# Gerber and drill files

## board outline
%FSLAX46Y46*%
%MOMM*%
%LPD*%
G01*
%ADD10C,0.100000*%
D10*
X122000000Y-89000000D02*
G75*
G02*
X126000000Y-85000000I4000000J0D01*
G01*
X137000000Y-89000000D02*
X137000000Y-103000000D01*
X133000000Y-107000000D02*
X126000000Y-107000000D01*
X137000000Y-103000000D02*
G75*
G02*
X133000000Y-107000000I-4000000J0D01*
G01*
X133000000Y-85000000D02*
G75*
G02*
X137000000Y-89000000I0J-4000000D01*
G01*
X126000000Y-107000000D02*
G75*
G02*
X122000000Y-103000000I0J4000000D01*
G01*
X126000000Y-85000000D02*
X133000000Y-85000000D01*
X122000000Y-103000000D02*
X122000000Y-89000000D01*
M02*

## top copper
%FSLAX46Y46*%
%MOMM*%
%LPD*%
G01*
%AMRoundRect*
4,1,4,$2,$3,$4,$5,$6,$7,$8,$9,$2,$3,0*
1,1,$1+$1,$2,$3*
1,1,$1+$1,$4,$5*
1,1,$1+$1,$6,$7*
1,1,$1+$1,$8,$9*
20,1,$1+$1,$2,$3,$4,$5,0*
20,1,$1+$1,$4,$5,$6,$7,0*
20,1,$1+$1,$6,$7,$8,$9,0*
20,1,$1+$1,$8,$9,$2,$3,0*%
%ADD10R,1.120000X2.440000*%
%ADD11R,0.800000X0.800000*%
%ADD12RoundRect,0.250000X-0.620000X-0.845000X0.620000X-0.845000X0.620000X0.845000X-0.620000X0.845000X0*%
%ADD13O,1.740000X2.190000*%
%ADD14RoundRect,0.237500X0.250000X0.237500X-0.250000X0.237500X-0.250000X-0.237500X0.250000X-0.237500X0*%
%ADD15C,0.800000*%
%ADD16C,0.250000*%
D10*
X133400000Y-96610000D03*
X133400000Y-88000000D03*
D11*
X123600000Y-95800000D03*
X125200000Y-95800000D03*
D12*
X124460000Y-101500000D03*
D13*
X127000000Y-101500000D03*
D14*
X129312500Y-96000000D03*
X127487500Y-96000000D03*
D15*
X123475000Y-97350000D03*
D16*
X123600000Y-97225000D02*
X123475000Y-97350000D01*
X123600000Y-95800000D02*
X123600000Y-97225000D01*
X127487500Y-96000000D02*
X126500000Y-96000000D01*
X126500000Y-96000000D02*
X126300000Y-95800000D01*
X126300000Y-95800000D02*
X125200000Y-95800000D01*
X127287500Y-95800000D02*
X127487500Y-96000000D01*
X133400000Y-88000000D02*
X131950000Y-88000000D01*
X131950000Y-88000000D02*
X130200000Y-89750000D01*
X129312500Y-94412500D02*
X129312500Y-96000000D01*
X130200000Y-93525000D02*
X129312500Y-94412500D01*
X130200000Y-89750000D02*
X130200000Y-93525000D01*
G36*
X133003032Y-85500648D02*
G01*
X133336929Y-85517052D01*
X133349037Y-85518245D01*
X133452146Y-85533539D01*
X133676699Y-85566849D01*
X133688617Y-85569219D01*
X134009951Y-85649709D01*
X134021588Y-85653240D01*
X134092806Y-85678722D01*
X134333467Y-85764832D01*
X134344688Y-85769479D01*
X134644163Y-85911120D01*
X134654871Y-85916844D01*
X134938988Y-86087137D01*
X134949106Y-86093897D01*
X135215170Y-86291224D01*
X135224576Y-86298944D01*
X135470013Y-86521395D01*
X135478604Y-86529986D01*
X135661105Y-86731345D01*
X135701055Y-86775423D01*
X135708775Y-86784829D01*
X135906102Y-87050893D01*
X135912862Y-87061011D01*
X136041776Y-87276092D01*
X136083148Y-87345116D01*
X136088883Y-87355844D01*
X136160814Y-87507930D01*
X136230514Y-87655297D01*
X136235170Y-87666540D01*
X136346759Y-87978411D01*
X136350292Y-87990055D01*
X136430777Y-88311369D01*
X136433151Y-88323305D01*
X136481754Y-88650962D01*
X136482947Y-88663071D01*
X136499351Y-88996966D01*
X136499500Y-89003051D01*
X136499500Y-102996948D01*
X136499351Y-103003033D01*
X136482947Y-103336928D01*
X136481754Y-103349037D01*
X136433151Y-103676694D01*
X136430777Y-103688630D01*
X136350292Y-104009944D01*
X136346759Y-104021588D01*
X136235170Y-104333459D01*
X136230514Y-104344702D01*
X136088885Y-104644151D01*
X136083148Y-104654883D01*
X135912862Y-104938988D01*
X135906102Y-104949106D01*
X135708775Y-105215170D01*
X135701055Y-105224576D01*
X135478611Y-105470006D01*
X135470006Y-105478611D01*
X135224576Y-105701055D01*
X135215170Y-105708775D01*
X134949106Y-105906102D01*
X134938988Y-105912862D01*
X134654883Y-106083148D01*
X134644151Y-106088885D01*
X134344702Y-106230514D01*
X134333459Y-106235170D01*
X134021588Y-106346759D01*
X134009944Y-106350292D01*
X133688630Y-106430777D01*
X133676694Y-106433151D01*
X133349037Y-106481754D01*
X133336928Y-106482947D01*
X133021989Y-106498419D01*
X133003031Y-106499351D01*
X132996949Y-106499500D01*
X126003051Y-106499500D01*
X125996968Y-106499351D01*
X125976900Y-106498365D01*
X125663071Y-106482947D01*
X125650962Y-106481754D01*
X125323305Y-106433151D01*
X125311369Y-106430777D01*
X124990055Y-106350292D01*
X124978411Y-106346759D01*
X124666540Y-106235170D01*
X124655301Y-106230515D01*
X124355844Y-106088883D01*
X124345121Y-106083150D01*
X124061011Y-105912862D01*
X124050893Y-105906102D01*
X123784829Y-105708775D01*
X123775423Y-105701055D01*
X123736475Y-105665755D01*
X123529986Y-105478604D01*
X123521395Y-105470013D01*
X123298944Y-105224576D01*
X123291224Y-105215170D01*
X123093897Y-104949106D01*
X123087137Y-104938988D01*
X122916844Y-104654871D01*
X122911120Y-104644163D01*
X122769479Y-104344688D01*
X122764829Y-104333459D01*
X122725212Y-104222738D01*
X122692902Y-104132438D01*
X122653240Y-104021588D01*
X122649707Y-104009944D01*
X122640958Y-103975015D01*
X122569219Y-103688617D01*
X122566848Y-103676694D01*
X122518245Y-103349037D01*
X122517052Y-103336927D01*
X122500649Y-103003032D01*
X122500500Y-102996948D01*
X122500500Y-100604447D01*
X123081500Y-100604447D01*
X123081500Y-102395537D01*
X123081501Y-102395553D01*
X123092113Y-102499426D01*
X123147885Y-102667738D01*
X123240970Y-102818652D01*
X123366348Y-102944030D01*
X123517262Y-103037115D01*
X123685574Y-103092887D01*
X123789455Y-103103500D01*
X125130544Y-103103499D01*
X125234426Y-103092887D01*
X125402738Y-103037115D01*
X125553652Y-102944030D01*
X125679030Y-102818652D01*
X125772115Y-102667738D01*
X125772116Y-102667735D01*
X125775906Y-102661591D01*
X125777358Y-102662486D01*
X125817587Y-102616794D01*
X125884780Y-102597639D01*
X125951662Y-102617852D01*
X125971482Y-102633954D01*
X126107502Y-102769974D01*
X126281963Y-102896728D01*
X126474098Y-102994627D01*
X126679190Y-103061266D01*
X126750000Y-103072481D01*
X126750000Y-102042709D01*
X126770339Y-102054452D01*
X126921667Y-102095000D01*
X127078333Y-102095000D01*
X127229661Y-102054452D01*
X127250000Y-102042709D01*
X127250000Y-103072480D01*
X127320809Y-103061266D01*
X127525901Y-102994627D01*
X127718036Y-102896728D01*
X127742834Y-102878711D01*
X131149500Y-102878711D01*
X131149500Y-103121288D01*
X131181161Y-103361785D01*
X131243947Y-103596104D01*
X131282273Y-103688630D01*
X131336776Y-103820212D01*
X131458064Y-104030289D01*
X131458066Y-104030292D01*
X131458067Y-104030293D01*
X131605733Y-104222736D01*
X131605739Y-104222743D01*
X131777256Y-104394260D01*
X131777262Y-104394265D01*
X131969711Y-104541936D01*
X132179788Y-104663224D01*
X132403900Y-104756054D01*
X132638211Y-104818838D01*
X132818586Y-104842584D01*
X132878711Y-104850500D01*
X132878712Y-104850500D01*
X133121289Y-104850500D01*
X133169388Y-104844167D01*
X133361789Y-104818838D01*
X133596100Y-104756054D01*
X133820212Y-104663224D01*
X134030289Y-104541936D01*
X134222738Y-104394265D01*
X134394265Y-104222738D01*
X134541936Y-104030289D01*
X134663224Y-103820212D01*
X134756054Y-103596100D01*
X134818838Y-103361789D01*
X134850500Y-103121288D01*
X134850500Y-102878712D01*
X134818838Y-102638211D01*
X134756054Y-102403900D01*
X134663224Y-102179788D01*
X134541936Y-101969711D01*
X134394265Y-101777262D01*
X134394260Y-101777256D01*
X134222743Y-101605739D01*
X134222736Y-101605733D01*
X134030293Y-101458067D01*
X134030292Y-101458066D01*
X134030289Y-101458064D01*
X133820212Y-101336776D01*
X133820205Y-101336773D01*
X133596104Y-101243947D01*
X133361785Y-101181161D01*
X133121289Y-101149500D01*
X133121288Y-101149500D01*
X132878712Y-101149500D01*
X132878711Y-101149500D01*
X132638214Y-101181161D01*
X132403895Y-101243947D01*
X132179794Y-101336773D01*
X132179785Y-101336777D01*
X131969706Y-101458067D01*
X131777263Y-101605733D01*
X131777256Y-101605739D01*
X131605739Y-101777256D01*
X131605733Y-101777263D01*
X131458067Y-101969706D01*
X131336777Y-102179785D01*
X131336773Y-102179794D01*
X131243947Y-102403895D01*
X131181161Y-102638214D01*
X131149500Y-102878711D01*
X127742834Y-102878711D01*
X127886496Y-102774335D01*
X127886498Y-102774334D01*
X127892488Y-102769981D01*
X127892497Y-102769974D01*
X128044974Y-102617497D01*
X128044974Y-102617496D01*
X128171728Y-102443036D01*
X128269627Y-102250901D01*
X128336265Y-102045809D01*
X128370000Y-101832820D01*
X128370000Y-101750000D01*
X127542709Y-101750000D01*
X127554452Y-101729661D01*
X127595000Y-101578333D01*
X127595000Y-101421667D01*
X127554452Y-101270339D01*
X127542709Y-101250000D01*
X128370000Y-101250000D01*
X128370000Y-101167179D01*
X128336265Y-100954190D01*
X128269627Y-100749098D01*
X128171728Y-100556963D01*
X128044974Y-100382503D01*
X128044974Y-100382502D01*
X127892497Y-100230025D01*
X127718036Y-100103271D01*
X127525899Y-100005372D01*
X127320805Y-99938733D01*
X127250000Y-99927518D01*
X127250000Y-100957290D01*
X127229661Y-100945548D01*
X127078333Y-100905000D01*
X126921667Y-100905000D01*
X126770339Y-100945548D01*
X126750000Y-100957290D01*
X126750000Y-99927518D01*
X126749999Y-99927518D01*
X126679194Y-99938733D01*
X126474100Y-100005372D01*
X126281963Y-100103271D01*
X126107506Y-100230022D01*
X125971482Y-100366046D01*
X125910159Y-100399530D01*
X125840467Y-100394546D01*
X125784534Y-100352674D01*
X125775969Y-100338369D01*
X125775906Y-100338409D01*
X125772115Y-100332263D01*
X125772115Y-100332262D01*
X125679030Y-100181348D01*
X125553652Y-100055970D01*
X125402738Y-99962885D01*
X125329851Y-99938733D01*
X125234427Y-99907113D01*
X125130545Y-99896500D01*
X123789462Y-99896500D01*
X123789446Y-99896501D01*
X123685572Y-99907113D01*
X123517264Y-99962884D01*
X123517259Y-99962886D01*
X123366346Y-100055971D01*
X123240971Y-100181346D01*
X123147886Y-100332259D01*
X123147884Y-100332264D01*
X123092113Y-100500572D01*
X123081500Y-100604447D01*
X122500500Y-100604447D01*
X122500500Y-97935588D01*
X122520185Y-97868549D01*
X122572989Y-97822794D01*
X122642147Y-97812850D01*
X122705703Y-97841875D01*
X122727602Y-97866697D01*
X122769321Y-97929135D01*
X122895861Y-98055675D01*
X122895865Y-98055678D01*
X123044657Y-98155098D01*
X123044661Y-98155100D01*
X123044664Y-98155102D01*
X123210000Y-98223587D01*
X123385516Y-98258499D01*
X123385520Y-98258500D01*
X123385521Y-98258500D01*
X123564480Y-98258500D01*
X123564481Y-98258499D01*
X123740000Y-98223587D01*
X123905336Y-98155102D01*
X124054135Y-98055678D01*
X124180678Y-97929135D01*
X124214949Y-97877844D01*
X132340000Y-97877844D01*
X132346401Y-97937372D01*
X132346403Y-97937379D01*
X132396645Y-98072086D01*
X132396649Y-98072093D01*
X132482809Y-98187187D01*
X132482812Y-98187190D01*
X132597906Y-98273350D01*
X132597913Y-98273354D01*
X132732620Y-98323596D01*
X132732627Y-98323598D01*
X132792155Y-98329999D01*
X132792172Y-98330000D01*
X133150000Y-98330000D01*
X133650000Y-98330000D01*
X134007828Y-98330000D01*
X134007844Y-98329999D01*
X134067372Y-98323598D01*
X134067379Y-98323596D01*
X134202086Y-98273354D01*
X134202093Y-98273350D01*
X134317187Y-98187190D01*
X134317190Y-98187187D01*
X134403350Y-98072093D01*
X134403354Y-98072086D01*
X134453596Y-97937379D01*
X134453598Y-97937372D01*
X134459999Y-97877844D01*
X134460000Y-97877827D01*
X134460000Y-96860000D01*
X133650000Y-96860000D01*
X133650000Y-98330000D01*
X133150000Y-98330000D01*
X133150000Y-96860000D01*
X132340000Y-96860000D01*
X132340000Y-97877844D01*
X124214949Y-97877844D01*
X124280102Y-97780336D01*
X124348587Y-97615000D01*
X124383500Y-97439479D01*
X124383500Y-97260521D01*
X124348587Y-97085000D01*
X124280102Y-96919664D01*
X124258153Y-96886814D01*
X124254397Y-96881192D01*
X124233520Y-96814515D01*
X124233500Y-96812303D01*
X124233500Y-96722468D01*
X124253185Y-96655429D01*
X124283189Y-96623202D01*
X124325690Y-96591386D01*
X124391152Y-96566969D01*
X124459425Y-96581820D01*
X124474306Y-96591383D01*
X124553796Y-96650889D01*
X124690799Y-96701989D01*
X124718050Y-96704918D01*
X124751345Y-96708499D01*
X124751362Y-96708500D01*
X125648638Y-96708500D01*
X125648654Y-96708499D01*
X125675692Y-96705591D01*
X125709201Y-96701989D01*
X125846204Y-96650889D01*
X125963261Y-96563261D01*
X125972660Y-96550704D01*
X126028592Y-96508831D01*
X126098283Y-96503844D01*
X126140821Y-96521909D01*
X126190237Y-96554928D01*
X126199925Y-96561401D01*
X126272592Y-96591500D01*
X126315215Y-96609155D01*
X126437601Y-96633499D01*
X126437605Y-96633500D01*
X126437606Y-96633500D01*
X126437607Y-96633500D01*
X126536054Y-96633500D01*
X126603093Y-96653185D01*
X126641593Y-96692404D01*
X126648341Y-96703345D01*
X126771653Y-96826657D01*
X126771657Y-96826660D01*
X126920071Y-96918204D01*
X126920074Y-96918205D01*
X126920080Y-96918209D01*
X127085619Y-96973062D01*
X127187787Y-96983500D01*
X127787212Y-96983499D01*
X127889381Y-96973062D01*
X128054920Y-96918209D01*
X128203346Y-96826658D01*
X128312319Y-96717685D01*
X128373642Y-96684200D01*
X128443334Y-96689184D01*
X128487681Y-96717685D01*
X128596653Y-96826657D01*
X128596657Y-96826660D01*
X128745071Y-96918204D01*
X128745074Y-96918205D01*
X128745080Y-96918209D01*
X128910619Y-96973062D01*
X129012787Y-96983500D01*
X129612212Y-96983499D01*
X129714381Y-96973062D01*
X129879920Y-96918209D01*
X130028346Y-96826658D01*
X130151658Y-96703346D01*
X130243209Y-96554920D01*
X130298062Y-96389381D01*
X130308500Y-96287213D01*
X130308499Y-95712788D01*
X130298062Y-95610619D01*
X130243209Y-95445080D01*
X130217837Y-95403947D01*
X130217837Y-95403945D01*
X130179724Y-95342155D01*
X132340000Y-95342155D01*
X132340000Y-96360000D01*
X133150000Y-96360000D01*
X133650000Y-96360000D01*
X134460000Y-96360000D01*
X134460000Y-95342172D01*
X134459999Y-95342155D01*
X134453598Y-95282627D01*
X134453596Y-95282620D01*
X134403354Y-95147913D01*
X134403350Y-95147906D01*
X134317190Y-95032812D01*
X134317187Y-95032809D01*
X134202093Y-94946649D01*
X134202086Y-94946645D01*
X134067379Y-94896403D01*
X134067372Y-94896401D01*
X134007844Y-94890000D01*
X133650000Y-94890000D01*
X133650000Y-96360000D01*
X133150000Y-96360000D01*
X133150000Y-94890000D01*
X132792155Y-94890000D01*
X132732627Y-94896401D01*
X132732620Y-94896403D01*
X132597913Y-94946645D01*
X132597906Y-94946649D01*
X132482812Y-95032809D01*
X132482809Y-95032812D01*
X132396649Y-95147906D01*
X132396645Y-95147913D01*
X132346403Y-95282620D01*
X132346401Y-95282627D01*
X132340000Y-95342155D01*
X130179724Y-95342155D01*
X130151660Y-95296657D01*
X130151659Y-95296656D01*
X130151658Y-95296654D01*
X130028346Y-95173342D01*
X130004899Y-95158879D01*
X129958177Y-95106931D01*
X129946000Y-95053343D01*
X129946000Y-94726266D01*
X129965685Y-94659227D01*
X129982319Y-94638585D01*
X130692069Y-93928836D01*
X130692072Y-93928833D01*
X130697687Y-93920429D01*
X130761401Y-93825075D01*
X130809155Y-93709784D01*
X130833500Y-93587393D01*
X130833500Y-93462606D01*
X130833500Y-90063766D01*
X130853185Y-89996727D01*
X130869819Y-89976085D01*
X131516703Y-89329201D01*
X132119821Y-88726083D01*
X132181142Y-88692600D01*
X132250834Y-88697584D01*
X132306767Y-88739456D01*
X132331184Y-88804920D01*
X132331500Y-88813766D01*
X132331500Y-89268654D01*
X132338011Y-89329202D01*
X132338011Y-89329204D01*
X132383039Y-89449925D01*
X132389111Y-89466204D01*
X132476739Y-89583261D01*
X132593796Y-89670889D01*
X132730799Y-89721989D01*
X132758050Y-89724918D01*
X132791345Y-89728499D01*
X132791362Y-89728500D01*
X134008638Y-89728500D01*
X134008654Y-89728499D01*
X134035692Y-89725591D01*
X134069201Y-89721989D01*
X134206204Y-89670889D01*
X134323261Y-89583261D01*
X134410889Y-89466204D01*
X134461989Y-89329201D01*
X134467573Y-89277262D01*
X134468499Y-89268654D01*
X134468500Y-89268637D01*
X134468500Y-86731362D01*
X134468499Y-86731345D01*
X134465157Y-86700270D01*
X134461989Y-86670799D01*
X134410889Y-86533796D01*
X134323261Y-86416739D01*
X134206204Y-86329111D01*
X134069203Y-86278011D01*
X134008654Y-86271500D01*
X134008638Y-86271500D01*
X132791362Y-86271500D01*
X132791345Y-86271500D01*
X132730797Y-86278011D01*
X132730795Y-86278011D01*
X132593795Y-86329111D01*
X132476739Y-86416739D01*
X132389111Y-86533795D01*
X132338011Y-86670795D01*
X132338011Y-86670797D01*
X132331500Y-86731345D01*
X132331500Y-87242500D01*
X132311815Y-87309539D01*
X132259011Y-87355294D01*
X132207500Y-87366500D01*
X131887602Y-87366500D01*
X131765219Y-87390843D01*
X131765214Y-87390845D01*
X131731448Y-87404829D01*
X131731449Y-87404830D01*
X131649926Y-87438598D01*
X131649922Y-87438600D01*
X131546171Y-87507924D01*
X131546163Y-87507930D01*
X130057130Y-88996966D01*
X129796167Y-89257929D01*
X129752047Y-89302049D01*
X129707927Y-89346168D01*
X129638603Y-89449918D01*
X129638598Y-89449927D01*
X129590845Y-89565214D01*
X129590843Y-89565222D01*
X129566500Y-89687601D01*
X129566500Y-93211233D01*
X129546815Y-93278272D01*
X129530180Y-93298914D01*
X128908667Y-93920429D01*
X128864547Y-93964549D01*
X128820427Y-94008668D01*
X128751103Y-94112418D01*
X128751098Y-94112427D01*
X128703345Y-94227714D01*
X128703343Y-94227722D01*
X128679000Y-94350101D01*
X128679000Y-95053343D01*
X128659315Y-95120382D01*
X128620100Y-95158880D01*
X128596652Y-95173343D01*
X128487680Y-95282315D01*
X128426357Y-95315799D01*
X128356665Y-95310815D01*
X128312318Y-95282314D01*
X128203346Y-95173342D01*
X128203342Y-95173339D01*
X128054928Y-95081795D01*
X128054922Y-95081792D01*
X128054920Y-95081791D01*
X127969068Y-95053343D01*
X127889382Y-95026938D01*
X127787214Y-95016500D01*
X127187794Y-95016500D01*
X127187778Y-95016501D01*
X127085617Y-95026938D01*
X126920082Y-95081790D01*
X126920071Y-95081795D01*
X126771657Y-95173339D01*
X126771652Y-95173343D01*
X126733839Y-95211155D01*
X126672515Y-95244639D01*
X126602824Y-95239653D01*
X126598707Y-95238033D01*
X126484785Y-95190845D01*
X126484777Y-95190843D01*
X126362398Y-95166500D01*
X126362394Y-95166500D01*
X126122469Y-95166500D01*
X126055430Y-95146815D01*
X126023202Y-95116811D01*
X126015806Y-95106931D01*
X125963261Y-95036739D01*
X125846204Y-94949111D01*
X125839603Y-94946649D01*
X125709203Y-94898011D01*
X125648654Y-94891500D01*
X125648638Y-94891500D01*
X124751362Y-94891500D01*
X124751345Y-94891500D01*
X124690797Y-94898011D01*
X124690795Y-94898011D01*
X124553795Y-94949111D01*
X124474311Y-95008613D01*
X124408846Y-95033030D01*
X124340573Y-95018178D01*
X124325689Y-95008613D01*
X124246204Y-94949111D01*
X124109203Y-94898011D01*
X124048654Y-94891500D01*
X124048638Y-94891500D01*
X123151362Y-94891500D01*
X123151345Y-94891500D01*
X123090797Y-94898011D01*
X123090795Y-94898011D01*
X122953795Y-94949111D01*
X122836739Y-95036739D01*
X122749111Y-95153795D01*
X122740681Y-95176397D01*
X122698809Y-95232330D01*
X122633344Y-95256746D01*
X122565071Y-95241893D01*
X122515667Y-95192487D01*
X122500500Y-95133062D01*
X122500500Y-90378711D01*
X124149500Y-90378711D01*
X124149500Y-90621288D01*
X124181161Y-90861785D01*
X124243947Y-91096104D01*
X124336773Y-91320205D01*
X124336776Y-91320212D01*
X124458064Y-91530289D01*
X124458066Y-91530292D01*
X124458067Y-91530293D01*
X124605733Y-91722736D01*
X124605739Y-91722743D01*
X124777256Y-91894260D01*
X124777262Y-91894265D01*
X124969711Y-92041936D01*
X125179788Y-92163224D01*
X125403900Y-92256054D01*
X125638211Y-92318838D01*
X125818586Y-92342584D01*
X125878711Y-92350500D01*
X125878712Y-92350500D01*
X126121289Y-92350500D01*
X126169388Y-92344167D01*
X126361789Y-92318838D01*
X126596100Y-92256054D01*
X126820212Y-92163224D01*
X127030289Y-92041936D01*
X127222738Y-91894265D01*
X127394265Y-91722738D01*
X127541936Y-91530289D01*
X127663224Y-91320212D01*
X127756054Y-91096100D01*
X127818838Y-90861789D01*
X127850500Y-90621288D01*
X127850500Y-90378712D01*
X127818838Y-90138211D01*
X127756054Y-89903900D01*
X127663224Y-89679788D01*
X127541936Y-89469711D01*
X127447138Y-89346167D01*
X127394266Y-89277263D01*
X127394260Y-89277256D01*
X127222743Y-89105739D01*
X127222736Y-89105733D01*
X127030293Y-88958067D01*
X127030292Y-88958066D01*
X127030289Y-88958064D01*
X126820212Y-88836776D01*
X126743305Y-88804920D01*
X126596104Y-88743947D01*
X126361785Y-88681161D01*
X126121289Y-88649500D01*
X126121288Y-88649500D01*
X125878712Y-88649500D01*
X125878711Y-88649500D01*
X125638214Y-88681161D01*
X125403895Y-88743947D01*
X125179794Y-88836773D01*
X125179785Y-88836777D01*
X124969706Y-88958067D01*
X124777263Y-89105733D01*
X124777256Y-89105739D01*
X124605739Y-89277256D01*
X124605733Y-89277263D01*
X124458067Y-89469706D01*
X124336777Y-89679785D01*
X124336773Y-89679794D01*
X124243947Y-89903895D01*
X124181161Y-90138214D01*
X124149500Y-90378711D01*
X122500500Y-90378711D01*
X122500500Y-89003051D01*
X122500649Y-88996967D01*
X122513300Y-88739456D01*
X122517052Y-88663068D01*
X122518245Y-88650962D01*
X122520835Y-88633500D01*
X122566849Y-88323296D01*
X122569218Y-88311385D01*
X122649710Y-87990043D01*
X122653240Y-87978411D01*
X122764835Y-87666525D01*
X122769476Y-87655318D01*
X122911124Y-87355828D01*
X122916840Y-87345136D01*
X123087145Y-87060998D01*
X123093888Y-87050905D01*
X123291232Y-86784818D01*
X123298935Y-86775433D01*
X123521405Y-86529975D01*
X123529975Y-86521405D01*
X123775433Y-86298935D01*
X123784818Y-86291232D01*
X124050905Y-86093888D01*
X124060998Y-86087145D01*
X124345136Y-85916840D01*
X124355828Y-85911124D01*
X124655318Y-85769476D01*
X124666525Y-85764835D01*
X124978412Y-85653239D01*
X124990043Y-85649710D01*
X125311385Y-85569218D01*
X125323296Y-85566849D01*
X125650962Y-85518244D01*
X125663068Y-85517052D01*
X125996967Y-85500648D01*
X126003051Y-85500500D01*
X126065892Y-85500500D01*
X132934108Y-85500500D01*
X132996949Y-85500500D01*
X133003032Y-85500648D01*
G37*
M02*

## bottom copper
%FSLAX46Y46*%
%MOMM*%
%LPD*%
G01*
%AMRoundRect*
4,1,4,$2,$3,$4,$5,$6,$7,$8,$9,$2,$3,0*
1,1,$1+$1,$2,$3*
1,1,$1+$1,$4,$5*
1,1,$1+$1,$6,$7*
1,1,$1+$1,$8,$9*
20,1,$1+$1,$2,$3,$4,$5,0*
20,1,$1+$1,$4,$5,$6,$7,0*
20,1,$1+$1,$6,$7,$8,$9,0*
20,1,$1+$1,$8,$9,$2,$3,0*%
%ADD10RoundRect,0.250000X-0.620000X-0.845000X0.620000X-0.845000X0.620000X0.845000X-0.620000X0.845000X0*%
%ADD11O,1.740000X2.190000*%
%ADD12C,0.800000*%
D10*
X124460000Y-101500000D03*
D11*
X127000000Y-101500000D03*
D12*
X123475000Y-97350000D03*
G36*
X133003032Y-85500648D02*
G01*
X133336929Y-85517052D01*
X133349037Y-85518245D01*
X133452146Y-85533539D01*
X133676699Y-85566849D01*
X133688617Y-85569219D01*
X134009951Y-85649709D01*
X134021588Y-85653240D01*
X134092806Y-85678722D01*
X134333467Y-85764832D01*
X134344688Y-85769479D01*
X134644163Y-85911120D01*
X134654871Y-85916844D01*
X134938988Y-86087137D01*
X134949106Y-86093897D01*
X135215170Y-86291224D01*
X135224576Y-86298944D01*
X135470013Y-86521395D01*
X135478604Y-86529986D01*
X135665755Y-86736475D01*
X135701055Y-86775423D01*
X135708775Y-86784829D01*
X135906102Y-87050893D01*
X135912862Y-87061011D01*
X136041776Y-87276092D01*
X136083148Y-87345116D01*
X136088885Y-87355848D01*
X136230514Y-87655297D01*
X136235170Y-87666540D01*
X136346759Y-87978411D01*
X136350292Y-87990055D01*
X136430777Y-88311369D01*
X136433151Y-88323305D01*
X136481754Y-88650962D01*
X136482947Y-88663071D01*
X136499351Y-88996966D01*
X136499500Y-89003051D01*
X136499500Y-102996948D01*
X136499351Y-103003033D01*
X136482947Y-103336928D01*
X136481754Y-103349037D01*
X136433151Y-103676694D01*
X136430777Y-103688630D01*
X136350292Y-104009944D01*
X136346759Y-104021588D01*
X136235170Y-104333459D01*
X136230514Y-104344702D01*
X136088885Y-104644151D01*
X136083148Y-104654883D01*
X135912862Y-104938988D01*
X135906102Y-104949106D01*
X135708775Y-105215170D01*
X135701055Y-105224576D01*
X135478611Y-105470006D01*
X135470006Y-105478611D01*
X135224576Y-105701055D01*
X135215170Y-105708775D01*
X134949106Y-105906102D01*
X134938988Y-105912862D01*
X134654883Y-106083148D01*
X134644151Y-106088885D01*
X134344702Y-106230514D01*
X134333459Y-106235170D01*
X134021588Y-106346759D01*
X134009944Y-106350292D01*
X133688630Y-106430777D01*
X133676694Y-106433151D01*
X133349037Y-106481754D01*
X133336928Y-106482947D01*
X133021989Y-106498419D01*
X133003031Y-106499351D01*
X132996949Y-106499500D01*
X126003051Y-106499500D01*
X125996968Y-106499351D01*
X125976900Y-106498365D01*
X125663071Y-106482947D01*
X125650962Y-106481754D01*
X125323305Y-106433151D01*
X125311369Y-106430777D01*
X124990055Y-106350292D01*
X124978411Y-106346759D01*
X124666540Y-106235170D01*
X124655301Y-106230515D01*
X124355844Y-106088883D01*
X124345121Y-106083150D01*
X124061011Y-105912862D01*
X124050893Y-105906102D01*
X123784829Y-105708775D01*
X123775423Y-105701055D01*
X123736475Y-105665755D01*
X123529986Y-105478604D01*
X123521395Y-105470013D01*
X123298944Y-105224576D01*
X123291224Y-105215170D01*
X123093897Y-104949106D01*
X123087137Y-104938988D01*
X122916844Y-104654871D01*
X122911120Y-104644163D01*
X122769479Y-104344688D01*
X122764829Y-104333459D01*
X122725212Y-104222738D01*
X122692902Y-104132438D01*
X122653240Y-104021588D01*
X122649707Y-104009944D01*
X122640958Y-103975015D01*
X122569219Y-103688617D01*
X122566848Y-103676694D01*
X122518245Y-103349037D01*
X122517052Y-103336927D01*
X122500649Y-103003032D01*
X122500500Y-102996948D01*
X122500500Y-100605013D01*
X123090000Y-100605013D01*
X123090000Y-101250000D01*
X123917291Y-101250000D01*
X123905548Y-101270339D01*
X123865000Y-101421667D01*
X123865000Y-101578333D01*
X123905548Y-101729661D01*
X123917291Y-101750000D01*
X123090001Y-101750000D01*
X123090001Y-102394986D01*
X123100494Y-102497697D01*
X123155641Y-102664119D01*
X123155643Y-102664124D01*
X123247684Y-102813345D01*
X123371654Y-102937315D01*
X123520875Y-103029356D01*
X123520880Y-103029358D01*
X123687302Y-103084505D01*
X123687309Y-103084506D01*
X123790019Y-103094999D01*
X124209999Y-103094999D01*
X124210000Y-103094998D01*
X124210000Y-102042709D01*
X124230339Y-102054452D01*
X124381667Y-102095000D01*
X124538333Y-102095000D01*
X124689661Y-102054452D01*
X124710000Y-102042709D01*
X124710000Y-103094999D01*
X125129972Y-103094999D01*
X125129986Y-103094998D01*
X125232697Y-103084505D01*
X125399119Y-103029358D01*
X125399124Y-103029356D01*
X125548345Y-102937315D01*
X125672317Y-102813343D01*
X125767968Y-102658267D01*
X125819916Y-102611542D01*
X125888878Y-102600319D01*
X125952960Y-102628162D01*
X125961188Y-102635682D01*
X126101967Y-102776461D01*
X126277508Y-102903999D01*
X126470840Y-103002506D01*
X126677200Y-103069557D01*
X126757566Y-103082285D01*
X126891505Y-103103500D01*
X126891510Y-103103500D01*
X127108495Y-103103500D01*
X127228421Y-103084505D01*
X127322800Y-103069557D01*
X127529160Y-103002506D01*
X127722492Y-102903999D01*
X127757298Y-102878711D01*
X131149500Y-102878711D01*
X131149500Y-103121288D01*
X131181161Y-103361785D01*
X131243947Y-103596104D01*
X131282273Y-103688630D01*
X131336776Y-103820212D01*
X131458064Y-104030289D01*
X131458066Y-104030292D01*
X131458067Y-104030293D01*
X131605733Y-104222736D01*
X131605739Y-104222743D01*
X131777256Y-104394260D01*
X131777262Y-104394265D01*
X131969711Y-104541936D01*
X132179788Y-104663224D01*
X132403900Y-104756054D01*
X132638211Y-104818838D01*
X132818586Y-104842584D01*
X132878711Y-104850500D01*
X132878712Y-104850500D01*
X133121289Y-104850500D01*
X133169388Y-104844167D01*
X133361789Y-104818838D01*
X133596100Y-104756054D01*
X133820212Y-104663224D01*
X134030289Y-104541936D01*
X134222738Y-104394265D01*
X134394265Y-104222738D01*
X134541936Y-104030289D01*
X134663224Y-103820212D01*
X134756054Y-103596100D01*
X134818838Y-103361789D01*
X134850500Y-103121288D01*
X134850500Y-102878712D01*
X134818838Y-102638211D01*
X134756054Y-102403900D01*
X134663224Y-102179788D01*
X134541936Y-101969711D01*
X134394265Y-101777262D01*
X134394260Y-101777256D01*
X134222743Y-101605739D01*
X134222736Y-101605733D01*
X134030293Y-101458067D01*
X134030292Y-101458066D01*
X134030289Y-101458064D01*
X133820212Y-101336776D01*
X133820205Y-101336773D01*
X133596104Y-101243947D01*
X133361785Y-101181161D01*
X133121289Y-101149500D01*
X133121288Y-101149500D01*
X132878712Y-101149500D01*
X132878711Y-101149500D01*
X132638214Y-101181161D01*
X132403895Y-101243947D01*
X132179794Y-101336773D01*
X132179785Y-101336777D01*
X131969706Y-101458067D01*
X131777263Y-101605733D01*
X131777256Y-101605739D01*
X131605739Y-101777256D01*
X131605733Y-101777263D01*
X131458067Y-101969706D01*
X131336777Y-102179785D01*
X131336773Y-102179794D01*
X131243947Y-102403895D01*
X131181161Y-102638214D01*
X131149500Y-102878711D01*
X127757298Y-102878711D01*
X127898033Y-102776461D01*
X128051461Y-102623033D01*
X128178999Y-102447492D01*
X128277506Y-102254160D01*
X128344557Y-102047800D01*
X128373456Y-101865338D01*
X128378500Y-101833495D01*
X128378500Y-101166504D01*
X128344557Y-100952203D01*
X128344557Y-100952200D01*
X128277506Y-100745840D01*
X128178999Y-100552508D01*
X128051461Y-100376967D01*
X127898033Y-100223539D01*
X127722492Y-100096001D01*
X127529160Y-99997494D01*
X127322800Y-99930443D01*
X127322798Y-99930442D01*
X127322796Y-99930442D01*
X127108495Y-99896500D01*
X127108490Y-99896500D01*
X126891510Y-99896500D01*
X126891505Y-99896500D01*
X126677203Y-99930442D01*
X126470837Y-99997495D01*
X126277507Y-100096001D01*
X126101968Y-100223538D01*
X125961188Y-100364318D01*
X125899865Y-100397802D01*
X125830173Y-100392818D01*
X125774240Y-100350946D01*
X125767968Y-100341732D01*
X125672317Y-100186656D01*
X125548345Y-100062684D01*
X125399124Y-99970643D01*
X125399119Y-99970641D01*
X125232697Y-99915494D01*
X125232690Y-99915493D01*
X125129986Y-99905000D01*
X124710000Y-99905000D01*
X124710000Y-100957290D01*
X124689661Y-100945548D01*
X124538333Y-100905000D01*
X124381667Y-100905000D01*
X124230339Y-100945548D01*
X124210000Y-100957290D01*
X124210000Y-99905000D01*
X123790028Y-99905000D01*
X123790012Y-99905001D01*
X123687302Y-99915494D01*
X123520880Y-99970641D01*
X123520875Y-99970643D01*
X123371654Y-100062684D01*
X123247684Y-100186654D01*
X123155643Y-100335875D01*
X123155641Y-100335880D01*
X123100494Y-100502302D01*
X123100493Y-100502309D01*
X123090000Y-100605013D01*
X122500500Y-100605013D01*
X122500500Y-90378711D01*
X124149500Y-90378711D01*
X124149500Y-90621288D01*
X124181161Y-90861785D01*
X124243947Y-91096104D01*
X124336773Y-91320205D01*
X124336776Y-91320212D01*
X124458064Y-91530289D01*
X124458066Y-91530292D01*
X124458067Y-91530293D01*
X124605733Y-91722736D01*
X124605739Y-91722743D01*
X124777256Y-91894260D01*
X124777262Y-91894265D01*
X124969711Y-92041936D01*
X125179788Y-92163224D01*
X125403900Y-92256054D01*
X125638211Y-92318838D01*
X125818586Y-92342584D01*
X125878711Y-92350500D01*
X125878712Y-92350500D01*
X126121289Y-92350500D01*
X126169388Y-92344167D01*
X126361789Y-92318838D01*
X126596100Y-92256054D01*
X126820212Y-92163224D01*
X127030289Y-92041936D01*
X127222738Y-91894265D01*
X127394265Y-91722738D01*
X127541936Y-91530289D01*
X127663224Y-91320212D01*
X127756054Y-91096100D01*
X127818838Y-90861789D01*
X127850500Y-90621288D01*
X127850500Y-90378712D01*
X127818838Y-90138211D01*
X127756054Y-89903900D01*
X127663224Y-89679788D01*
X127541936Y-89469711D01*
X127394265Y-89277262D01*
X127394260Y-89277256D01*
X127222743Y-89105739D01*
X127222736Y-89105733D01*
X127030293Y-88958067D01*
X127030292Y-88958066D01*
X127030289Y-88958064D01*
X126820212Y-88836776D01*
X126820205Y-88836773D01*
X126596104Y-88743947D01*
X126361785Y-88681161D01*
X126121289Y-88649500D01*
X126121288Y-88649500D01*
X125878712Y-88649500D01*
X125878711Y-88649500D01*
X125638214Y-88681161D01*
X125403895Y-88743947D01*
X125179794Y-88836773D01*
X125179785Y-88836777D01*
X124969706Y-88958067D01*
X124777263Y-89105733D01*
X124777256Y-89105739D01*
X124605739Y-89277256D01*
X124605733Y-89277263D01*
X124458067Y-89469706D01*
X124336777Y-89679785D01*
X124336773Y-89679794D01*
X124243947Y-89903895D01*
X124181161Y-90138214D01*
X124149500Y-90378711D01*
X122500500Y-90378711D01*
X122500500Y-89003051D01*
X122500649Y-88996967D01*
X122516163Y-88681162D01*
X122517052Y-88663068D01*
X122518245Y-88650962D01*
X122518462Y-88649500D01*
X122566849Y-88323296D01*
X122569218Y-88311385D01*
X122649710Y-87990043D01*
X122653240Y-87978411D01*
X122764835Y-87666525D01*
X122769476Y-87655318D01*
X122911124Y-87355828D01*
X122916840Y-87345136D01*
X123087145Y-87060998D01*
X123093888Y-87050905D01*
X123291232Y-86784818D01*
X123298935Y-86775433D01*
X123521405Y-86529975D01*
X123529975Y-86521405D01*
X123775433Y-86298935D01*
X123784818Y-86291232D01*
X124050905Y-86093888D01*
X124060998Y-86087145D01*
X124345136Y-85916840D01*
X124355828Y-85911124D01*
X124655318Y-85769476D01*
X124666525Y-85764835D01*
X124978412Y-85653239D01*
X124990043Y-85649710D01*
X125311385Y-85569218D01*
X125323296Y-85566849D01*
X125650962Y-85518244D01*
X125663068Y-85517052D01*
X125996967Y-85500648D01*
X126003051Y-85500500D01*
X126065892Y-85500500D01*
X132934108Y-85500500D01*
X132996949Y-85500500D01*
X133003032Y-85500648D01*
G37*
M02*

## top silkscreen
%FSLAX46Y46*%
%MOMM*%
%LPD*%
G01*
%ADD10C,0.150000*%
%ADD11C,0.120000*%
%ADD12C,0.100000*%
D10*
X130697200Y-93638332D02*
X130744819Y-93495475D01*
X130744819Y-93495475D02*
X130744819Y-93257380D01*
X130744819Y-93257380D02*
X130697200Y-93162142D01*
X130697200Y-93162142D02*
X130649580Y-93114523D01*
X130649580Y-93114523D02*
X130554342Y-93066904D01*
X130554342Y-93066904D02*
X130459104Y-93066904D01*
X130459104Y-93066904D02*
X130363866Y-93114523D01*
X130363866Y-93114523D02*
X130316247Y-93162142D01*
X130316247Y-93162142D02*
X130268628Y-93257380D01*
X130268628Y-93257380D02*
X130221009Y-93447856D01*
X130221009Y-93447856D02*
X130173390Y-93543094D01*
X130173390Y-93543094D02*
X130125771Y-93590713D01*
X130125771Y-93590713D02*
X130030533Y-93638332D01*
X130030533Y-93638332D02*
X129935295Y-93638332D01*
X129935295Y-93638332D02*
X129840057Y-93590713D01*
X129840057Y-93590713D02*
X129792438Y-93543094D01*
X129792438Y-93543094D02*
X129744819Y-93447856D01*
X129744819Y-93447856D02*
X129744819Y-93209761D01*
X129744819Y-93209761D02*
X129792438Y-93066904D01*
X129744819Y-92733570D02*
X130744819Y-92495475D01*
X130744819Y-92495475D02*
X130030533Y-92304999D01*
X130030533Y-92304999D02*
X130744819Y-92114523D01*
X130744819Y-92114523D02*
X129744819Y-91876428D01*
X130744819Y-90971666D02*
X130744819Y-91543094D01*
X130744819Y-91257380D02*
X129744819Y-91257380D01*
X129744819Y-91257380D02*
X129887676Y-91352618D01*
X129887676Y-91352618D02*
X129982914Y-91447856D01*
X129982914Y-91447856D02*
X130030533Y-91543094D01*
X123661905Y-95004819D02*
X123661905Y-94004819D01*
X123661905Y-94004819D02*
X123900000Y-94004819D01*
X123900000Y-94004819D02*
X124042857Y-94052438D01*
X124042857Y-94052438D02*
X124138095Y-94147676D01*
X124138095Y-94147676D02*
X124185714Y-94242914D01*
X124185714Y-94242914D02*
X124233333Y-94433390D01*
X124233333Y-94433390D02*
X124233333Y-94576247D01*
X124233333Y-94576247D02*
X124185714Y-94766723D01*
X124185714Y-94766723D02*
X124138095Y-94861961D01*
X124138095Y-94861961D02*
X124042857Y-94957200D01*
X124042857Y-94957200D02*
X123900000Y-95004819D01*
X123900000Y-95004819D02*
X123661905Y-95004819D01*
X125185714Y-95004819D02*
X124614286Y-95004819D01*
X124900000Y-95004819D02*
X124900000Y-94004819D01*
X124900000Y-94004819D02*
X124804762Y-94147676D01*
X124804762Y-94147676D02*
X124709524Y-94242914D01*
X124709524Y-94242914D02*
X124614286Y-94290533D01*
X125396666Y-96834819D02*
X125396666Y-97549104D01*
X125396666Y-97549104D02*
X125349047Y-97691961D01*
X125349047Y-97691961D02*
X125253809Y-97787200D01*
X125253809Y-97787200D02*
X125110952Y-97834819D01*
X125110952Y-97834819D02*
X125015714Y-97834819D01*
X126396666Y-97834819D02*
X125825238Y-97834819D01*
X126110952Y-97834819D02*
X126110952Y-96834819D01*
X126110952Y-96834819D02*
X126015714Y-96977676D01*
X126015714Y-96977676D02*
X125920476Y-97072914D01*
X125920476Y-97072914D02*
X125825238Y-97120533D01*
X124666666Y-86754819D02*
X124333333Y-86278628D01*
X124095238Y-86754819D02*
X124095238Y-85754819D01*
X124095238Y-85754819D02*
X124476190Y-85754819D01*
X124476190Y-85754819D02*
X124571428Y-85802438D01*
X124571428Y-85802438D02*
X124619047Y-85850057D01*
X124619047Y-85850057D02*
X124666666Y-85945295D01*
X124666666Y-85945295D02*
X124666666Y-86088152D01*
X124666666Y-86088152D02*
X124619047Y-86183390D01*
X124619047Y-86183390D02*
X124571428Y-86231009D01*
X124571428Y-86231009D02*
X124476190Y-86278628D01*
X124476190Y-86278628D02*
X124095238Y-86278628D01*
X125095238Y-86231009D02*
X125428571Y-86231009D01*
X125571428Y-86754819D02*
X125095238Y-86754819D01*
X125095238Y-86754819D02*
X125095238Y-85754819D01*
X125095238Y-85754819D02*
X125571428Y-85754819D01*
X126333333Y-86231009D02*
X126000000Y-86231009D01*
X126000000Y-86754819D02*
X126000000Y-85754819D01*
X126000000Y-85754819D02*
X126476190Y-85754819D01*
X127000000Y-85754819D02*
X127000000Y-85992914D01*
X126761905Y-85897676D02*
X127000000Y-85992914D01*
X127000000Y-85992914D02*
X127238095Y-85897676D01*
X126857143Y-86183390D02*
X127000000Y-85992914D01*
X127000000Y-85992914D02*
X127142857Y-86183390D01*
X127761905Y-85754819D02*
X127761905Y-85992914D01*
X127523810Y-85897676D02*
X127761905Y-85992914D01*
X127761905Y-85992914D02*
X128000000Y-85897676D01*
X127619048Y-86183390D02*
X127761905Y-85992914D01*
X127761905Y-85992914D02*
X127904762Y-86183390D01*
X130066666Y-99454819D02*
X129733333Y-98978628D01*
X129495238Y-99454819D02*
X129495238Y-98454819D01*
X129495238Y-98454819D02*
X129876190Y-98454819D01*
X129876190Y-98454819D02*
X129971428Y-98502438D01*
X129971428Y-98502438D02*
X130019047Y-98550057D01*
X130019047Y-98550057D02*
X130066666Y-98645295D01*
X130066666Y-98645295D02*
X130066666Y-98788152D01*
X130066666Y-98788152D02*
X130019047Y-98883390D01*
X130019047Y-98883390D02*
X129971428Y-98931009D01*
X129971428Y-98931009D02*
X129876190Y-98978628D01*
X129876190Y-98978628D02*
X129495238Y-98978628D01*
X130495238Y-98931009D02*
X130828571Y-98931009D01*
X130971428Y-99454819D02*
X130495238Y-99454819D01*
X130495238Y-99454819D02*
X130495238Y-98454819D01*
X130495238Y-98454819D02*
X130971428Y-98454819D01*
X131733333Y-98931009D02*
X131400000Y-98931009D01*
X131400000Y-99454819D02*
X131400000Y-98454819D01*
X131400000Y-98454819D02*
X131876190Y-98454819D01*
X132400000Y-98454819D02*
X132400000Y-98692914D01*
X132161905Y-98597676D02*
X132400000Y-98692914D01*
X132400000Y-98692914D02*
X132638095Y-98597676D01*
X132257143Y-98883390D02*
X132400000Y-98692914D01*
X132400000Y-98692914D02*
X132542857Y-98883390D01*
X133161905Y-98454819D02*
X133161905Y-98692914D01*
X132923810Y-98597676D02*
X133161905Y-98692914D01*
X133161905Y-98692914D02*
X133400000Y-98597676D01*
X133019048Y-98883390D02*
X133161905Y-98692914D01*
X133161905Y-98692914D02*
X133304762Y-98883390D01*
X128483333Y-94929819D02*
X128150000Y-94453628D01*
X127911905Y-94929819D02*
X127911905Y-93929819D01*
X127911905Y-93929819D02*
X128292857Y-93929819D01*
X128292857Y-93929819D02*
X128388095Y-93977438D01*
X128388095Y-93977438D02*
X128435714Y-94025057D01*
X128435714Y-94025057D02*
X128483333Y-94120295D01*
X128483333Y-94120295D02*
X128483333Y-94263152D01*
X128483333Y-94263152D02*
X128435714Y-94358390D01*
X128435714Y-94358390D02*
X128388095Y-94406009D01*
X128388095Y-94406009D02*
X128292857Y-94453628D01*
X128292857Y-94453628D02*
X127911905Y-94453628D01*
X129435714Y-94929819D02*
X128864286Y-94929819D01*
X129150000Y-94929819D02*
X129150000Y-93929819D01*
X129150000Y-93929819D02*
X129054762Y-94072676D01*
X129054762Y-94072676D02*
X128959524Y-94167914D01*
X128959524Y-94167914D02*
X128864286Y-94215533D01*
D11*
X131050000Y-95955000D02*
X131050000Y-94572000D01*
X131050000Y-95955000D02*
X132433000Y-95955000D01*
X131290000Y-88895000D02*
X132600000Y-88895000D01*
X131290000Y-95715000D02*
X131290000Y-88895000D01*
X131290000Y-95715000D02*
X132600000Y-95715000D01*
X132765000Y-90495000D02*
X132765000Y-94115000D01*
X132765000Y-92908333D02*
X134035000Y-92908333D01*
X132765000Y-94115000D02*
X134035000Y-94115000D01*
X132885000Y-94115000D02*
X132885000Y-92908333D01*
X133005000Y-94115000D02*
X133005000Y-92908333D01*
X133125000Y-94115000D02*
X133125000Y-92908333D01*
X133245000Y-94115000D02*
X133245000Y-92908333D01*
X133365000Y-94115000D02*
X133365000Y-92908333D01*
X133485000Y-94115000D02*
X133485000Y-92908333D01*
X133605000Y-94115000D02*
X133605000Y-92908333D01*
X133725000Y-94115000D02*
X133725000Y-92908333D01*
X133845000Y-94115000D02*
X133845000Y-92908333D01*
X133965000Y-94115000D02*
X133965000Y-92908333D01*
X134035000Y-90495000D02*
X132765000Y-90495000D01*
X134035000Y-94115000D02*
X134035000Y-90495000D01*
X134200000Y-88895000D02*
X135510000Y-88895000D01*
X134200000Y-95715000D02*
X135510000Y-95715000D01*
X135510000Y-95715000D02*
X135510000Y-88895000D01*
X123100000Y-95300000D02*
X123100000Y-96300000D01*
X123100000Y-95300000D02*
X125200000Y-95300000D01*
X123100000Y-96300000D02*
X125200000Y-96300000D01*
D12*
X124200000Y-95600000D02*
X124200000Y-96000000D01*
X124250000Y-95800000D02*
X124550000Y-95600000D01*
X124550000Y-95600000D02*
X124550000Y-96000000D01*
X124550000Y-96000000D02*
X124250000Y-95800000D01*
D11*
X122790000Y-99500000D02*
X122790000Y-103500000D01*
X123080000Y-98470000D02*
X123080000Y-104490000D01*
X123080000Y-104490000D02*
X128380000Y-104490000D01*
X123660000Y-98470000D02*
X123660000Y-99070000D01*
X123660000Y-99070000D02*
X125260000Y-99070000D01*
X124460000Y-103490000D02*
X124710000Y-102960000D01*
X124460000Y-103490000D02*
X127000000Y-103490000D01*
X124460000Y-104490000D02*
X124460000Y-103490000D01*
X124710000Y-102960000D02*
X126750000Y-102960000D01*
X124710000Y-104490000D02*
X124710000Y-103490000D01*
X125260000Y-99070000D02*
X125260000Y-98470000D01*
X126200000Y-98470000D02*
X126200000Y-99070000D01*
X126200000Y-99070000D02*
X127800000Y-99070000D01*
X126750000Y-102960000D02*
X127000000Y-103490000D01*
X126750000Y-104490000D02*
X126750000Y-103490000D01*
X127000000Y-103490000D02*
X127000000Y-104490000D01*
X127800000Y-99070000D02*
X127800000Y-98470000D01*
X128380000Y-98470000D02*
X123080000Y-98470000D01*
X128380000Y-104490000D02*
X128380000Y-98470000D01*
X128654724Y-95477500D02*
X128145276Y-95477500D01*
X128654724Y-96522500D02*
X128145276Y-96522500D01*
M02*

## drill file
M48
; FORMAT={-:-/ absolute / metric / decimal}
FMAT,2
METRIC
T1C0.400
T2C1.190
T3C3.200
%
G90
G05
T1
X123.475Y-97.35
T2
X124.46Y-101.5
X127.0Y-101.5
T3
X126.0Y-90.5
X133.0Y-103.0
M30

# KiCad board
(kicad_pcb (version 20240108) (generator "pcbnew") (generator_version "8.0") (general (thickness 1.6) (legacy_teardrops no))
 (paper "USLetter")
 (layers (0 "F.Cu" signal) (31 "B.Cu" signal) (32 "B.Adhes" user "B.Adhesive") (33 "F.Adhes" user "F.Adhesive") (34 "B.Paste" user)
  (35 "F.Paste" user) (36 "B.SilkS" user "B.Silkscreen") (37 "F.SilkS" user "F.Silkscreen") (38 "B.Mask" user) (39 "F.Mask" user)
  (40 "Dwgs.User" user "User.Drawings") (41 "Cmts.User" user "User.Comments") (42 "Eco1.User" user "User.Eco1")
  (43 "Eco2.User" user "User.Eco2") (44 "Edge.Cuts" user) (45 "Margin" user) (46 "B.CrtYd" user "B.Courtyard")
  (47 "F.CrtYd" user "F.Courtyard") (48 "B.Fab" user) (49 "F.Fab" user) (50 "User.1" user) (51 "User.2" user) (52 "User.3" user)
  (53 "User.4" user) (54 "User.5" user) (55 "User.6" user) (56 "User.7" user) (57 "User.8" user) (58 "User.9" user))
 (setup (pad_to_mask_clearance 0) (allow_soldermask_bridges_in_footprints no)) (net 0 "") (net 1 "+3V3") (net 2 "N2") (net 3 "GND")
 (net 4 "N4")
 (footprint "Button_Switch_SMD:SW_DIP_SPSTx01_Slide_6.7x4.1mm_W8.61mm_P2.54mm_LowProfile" (layer "F.Cu") (at 133.4 92.305 90)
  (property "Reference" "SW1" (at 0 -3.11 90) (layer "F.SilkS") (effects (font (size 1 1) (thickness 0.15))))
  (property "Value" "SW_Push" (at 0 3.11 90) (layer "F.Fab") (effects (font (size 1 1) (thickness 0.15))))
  (fp_line (start -3.65 -2.35) (end -2.267 -2.35) (stroke (width 0.12) (type solid)) (layer "F.SilkS"))
  (fp_line (start -3.65 -2.35) (end -3.65 -0.967) (stroke (width 0.12) (type solid)) (layer "F.SilkS"))
  (fp_line (start 3.41 -2.11) (end 3.41 -0.8) (stroke (width 0.12) (type solid)) (layer "F.SilkS"))
  (fp_line (start -3.41 -2.11) (end 3.41 -2.11) (stroke (width 0.12) (type solid)) (layer "F.SilkS"))
  (fp_line (start -3.41 -2.11) (end -3.41 -0.8) (stroke (width 0.12) (type solid)) (layer "F.SilkS"))
  (fp_line (start 1.81 -0.635) (end -1.81 -0.635) (stroke (width 0.12) (type solid)) (layer "F.SilkS"))
  (fp_line (start -0.603333 -0.635) (end -0.603333 0.635) (stroke (width 0.12) (type solid)) (layer "F.SilkS"))
  (fp_line (start -1.81 -0.635) (end -1.81 0.635) (stroke (width 0.12) (type solid)) (layer "F.SilkS"))
  (fp_line (start -1.81 -0.515) (end -0.603333 -0.515) (stroke (width 0.12) (type solid)) (layer "F.SilkS"))
  (fp_line (start -1.81 -0.395) (end -0.603333 -0.395) (stroke (width 0.12) (type solid)) (layer "F.SilkS"))
  (fp_line (start -1.81 -0.275) (end -0.603333 -0.275) (stroke (width 0.12) (type solid)) (layer "F.SilkS"))
  (fp_line (start -1.81 -0.155) (end -0.603333 -0.155) (stroke (width 0.12) (type solid)) (layer "F.SilkS"))
  (fp_line (start -1.81 -0.035) (end -0.603333 -0.035) (stroke (width 0.12) (type solid)) (layer "F.SilkS"))
  (fp_line (start -1.81 0.085) (end -0.603333 0.085) (stroke (width 0.12) (type solid)) (layer "F.SilkS"))
  (fp_line (start -1.81 0.205) (end -0.603333 0.205) (stroke (width 0.12) (type solid)) (layer "F.SilkS"))
  (fp_line (start -1.81 0.325) (end -0.603333 0.325) (stroke (width 0.12) (type solid)) (layer "F.SilkS"))
  (fp_line (start -1.81 0.445) (end -0.603333 0.445) (stroke (width 0.12) (type solid)) (layer "F.SilkS"))
  (fp_line (start -1.81 0.565) (end -0.603333 0.565) (stroke (width 0.12) (type solid)) (layer "F.SilkS"))
  (fp_line (start 1.81 0.635) (end 1.81 -0.635) (stroke (width 0.12) (type solid)) (layer "F.SilkS"))
  (fp_line (start -1.81 0.635) (end 1.81 0.635) (stroke (width 0.12) (type solid)) (layer "F.SilkS"))
  (fp_line (start 3.41 0.8) (end 3.41 2.11) (stroke (width 0.12) (type solid)) (layer "F.SilkS"))
  (fp_line (start -3.41 0.8) (end -3.41 2.11) (stroke (width 0.12) (type solid)) (layer "F.SilkS"))
  (fp_line (start -3.41 2.11) (end 3.41 2.11) (stroke (width 0.12) (type solid)) (layer "F.SilkS"))
  (pad "1" smd rect (at -4.305 0 90) (size 2.44 1.12) (layers "F.Cu" "F.Paste" "F.Mask") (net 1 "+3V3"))
  (pad "2" smd rect (at 4.305 0 90) (size 2.44 1.12) (layers "F.Cu" "F.Paste" "F.Mask") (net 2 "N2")))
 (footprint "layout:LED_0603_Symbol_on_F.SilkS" (layer "F.Cu") (at 124.4 95.8)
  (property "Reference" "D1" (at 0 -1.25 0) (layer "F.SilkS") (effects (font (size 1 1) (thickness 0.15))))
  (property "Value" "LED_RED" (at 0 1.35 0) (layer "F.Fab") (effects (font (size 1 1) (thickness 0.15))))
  (fp_line (start -1.3 -0.5) (end -1.3 0.5) (stroke (width 0.12) (type solid)) (layer "F.SilkS"))
  (fp_line (start -1.3 -0.5) (end 0.8 -0.5) (stroke (width 0.12) (type solid)) (layer "F.SilkS"))
  (fp_line (start -1.3 0.5) (end 0.8 0.5) (stroke (width 0.12) (type solid)) (layer "F.SilkS"))
  (fp_line (start -0.2 -0.2) (end -0.2 0.2) (stroke (width 0.1) (type solid)) (layer "F.SilkS"))
  (fp_line (start -0.15 0) (end 0.15 -0.2) (stroke (width 0.1) (type solid)) (layer "F.SilkS"))
  (fp_line (start 0.15 -0.2) (end 0.15 0.2) (stroke (width 0.1) (type solid)) (layer "F.SilkS"))
  (fp_line (start 0.15 0.2) (end -0.15 0) (stroke (width 0.1) (type solid)) (layer "F.SilkS"))
  (pad "1" smd rect (at -0.8 0 180) (size 0.8 0.8) (layers "F.Cu" "F.Paste" "F.Mask") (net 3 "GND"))
  (pad "2" smd rect (at 0.8 0 180) (size 0.8 0.8) (layers "F.Cu" "F.Paste" "F.Mask") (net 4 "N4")))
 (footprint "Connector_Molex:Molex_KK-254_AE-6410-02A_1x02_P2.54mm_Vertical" (layer "F.Cu") (at 124.46 101.5)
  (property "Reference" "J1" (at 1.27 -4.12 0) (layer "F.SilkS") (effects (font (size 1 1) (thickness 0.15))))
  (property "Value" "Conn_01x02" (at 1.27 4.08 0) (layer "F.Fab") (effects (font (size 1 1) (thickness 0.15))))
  (fp_line (start -1.67 -2) (end -1.67 2) (stroke (width 0.12) (type solid)) (layer "F.SilkS"))
  (fp_line (start -1.38 -3.03) (end -1.38 2.99) (stroke (width 0.12) (type solid)) (layer "F.SilkS"))
  (fp_line (start -1.38 2.99) (end 3.92 2.99) (stroke (width 0.12) (type solid)) (layer "F.SilkS"))
  (fp_line (start -0.8 -3.03) (end -0.8 -2.43) (stroke (width 0.12) (type solid)) (layer "F.SilkS"))
  (fp_line (start -0.8 -2.43) (end 0.8 -2.43) (stroke (width 0.12) (type solid)) (layer "F.SilkS"))
  (fp_line (start 0 1.99) (end 0.25 1.46) (stroke (width 0.12) (type solid)) (layer "F.SilkS"))
  (fp_line (start 0 1.99) (end 2.54 1.99) (stroke (width 0.12) (type solid)) (layer "F.SilkS"))
  (fp_line (start 0 2.99) (end 0 1.99) (stroke (width 0.12) (type solid)) (layer "F.SilkS"))
  (fp_line (start 0.25 1.46) (end 2.29 1.46) (stroke (width 0.12) (type solid)) (layer "F.SilkS"))
  (fp_line (start 0.25 2.99) (end 0.25 1.99) (stroke (width 0.12) (type solid)) (layer "F.SilkS"))
  (fp_line (start 0.8 -2.43) (end 0.8 -3.03) (stroke (width 0.12) (type solid)) (layer "F.SilkS"))
  (fp_line (start 1.74 -3.03) (end 1.74 -2.43) (stroke (width 0.12) (type solid)) (layer "F.SilkS"))
  (fp_line (start 1.74 -2.43) (end 3.34 -2.43) (stroke (width 0.12) (type solid)) (layer "F.SilkS"))
  (fp_line (start 2.29 1.46) (end 2.54 1.99) (stroke (width 0.12) (type solid)) (layer "F.SilkS"))
  (fp_line (start 2.29 2.99) (end 2.29 1.99) (stroke (width 0.12) (type solid)) (layer "F.SilkS"))
  (fp_line (start 2.54 1.99) (end 2.54 2.99) (stroke (width 0.12) (type solid)) (layer "F.SilkS"))
  (fp_line (start 3.34 -2.43) (end 3.34 -3.03) (stroke (width 0.12) (type solid)) (layer "F.SilkS"))
  (fp_line (start 3.92 -3.03) (end -1.38 -3.03) (stroke (width 0.12) (type solid)) (layer "F.SilkS"))
  (fp_line (start 3.92 2.99) (end 3.92 -3.03) (stroke (width 0.12) (type solid)) (layer "F.SilkS"))
  (pad "1" thru_hole roundrect (at 0 0) (size 1.74 2.19) (drill 1.19) (layers "*.Cu" "*.Mask") (remove_unused_layers no)
   (roundrect_rratio 0.143678) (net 3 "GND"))
  (pad "2" thru_hole oval (at 2.54 0) (size 1.74 2.19) (drill 1.19) (layers "*.Cu" "*.Mask") (remove_unused_layers no) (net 1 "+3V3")))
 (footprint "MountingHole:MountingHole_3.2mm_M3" (layer "F.Cu") (at 126 90.5)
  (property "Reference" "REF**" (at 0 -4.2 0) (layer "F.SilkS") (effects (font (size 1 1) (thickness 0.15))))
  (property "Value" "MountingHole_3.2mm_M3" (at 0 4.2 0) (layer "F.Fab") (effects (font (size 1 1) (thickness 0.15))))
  (pad "" np_thru_hole circle (at 0 0) (size 3.2 3.2) (drill 3.2) (layers "*.Cu" "*.Mask")))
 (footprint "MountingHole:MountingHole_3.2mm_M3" (layer "F.Cu") (at 133 103)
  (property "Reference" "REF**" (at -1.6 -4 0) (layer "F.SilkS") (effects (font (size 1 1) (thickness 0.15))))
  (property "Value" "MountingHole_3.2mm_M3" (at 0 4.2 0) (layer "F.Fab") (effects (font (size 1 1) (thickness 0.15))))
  (pad "" np_thru_hole circle (at 0 0) (size 3.2 3.2) (drill 3.2) (layers "*.Cu" "*.Mask")))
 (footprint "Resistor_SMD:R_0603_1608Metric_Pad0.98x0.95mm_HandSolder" (layer "F.Cu") (at 128.4 96 180)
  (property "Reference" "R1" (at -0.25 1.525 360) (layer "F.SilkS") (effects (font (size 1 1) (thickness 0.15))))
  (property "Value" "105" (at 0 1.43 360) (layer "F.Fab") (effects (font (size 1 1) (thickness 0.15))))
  (fp_line (start -0.254724 0.5225) (end 0.254724 0.5225) (stroke (width 0.12) (type solid)) (layer "F.SilkS"))
  (fp_line (start -0.254724 -0.5225) (end 0.254724 -0.5225) (stroke (width 0.12) (type solid)) (layer "F.SilkS"))
  (pad "1" smd roundrect (at -0.9125 0 180) (size 0.975 0.95) (layers "F.Cu" "F.Paste" "F.Mask") (roundrect_rratio 0.25) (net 2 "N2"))
  (pad "2" smd roundrect (at 0.9125 0 180) (size 0.975 0.95) (layers "F.Cu" "F.Paste" "F.Mask") (roundrect_rratio 0.25) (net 4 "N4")))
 (gr_arc (start 122 89) (mid 123.171573 86.171573) (end 126 85) (stroke (width 0.1) (type default)) (layer "Edge.Cuts"))
 (gr_line (start 137 89) (end 137 103) (stroke (width 0.1) (type default)) (layer "Edge.Cuts"))
 (gr_line (start 133 107) (end 126 107) (stroke (width 0.1) (type default)) (layer "Edge.Cuts"))
 (gr_arc (start 137 103) (mid 135.828427 105.828427) (end 133 107) (stroke (width 0.1) (type default)) (layer "Edge.Cuts"))
 (gr_arc (start 133 85) (mid 135.828427 86.171573) (end 137 89) (stroke (width 0.1) (type default)) (layer "Edge.Cuts"))
 (gr_arc (start 126 107) (mid 123.171573 105.828427) (end 122 103) (stroke (width 0.1) (type default)) (layer "Edge.Cuts"))
 (gr_line (start 126 85) (end 133 85) (stroke (width 0.1) (type default)) (layer "Edge.Cuts"))
 (gr_line (start 122 103) (end 122 89) (stroke (width 0.1) (type default)) (layer "Edge.Cuts"))
 (segment (start 123.6 97.225) (end 123.475 97.35) (width 0.25) (layer "F.Cu") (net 3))
 (segment (start 123.6 95.8) (end 123.6 97.225) (width 0.25) (layer "F.Cu") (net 3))
 (via (at 123.475 97.35) (size 0.8) (drill 0.4) (layers "F.Cu" "B.Cu") (free yes) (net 3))
 (segment (start 127.4875 96) (end 126.5 96) (width 0.25) (layer "F.Cu") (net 4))
 (segment (start 126.5 96) (end 126.3 95.8) (width 0.25) (layer "F.Cu") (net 4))
 (segment (start 126.3 95.8) (end 125.2 95.8) (width 0.25) (layer "F.Cu") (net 4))
 (segment (start 127.2875 95.8) (end 127.4875 96) (width 0.25) (layer "F.Cu") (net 4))
 (segment (start 133.4 88) (end 131.95 88) (width 0.25) (layer "F.Cu") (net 2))
 (segment (start 131.95 88) (end 130.2 89.75) (width 0.25) (layer "F.Cu") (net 2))
 (segment (start 129.3125 94.4125) (end 129.3125 96) (width 0.25) (layer "F.Cu") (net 2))
 (segment (start 130.2 93.525) (end 129.3125 94.4125) (width 0.25) (layer "F.Cu") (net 2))
 (segment (start 130.2 89.75) (end 130.2 93.525) (width 0.25) (layer "F.Cu") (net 2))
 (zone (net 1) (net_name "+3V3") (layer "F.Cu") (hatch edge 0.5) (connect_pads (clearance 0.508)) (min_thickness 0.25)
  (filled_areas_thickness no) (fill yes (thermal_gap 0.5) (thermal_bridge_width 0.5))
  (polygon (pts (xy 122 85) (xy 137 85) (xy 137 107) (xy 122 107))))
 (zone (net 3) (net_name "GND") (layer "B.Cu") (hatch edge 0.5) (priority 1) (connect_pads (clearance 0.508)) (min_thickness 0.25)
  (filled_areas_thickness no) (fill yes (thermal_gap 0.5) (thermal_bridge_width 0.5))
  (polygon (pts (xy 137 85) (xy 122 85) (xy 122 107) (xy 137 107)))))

